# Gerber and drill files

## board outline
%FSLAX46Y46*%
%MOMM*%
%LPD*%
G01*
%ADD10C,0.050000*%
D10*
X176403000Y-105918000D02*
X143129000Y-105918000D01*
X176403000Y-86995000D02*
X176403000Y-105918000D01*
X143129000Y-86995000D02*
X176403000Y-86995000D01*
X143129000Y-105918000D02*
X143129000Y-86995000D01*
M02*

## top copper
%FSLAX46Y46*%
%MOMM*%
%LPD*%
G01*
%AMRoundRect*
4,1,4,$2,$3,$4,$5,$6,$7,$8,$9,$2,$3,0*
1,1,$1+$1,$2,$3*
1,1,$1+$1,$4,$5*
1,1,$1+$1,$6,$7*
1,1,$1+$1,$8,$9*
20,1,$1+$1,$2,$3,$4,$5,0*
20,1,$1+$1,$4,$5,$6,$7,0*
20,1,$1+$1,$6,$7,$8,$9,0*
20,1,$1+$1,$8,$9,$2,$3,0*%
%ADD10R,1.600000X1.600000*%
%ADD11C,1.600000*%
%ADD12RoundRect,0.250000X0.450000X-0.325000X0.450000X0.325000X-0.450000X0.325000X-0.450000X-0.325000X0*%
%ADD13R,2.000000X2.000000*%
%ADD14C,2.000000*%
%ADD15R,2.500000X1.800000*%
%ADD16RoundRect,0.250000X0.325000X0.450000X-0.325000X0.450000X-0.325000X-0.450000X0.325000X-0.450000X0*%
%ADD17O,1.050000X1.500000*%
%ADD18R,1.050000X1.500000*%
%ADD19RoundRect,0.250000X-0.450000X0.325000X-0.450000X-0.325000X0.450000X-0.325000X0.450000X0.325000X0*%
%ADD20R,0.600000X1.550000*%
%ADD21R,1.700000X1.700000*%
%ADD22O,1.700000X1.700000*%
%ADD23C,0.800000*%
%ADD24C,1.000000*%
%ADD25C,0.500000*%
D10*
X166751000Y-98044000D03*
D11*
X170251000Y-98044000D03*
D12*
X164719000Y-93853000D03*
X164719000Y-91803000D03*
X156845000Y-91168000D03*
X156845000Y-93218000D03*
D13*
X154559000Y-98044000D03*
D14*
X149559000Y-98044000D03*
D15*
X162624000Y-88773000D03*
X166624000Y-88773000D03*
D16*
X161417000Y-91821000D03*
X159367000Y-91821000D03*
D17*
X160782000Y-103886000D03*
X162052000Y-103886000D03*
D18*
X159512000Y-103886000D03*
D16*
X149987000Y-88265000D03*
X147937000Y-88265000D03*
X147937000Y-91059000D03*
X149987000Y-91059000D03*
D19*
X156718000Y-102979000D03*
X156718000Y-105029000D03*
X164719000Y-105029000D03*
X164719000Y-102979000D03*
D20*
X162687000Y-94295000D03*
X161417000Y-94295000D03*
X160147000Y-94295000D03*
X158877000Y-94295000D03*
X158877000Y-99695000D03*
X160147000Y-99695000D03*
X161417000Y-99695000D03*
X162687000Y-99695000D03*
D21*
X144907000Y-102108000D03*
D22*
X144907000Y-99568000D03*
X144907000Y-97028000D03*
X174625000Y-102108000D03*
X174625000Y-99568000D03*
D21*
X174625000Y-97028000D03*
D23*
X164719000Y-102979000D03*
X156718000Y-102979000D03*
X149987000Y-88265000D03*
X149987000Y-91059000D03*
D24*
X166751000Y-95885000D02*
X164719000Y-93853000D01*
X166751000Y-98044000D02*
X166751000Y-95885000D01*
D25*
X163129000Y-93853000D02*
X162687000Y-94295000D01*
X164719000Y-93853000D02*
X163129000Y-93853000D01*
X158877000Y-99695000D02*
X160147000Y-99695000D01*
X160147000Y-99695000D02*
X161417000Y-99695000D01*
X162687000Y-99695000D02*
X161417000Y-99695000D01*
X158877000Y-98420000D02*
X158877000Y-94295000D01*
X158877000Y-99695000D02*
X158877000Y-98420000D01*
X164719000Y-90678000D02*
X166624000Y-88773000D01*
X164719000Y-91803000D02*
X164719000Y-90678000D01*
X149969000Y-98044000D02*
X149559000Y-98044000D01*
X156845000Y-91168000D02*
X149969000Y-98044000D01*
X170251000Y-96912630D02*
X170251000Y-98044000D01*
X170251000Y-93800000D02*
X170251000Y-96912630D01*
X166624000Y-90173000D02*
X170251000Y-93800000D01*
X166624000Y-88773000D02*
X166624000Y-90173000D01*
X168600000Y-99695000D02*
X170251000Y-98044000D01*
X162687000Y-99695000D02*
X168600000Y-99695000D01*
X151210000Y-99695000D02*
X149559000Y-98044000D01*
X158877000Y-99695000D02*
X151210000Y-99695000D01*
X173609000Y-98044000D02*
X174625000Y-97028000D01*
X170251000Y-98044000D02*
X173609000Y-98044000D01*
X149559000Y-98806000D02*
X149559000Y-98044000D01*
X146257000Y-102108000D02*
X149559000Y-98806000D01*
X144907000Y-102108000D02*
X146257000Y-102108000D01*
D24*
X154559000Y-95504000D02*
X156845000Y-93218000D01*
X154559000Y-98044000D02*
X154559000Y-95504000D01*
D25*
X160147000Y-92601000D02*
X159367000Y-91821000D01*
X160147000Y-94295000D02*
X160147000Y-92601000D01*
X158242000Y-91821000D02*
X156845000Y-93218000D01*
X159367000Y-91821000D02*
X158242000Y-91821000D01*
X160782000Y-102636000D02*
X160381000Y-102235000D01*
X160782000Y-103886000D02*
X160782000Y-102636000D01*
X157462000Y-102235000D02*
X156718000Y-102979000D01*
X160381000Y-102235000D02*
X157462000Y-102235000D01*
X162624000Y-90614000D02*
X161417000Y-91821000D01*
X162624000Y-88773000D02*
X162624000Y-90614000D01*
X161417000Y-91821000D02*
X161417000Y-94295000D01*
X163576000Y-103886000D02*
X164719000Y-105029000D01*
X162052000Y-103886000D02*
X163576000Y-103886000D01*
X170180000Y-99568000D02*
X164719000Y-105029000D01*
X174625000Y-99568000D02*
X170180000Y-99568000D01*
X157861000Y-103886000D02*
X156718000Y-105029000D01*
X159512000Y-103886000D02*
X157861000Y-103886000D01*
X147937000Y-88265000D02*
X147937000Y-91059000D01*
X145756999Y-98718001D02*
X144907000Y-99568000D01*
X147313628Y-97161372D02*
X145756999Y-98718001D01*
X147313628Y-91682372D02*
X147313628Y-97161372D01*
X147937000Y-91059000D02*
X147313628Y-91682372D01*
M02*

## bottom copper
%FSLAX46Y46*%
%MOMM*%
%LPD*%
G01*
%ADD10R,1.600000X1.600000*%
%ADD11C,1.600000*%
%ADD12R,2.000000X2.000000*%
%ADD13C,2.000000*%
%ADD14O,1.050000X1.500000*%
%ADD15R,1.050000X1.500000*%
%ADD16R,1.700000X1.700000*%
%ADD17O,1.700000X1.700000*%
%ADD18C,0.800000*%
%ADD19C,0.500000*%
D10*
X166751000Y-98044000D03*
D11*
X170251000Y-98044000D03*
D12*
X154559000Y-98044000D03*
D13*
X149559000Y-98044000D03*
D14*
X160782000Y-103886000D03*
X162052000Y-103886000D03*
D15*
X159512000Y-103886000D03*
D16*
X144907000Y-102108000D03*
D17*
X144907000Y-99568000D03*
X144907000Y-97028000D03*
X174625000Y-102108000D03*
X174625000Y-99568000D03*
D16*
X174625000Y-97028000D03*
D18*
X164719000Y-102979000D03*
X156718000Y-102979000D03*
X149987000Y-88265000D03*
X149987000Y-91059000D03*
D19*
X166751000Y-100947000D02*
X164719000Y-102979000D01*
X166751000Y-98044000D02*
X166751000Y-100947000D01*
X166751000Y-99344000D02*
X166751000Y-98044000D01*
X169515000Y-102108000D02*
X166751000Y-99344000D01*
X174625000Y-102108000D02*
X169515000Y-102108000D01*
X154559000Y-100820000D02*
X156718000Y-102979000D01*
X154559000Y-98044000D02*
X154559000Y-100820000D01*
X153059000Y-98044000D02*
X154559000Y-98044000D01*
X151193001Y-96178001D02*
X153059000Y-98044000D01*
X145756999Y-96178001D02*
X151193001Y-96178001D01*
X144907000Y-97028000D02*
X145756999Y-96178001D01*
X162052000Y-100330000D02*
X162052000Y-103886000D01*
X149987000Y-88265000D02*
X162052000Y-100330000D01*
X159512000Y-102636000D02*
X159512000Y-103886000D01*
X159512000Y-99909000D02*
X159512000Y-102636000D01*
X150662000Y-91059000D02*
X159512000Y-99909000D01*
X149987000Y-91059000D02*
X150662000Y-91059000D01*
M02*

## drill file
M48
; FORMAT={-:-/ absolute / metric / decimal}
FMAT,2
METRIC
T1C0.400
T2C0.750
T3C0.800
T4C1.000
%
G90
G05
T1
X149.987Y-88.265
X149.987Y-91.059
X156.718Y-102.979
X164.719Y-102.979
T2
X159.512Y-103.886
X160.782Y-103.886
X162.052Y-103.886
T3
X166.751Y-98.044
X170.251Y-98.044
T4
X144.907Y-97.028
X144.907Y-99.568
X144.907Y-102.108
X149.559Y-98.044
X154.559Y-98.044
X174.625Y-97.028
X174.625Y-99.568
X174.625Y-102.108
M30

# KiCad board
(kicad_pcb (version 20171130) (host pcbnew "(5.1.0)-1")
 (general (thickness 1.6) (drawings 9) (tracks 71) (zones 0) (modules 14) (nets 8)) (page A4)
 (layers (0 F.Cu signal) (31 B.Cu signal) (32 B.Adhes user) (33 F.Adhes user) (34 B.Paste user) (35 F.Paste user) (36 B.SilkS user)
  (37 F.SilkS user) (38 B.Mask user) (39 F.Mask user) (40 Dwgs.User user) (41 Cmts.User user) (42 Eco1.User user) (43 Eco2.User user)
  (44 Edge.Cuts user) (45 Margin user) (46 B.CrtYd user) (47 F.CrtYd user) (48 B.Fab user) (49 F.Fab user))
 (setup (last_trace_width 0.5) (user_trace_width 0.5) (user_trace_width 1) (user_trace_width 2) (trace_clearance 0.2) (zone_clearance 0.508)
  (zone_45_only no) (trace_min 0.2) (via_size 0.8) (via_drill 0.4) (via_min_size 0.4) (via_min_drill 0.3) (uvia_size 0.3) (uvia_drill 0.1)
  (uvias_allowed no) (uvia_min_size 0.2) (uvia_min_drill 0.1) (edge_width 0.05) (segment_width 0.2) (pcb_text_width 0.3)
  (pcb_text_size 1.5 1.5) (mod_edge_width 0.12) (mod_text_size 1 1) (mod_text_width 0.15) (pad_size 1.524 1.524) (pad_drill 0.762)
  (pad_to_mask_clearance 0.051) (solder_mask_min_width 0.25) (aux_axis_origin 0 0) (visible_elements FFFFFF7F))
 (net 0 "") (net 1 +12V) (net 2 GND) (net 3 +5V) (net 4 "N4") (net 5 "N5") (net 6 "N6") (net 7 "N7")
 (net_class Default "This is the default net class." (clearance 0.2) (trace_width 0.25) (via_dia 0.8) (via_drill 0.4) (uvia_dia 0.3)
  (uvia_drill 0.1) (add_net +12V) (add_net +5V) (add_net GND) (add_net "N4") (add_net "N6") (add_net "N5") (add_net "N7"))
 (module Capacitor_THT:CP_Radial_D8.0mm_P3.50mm (layer F.Cu) (at 166.751 98.044)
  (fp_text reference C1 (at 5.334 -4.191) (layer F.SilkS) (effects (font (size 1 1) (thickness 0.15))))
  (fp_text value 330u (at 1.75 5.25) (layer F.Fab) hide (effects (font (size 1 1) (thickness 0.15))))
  (pad 1 thru_hole rect (at 0 0) (size 1.6 1.6) (drill 0.8) (layers *.Cu *.Mask) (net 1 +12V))
  (pad 2 thru_hole circle (at 3.5 0) (size 1.6 1.6) (drill 0.8) (layers *.Cu *.Mask) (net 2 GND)))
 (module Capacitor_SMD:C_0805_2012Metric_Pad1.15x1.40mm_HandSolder (layer F.Cu) (at 164.719 92.828 90)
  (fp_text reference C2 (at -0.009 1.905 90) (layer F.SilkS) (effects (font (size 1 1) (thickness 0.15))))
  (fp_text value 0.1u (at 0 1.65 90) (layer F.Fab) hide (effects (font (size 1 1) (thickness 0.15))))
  (pad 1 smd roundrect (at -1.025 0 90) (size 1.15 1.4) (layers F.Cu F.Paste F.Mask) (roundrect_rratio 0.217391) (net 1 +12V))
  (pad 2 smd roundrect (at 1.025 0 90) (size 1.15 1.4) (layers F.Cu F.Paste F.Mask) (roundrect_rratio 0.217391) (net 2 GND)))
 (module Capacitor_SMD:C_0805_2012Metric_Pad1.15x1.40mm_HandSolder (layer F.Cu) (at 156.845 92.193 90)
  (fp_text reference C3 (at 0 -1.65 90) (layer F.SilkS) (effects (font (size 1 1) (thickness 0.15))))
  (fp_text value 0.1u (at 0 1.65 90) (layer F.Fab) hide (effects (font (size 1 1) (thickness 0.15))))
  (pad 2 smd roundrect (at 1.025 0 90) (size 1.15 1.4) (layers F.Cu F.Paste F.Mask) (roundrect_rratio 0.217391) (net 2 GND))
  (pad 1 smd roundrect (at -1.025 0 90) (size 1.15 1.4) (layers F.Cu F.Paste F.Mask) (roundrect_rratio 0.217391) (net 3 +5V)))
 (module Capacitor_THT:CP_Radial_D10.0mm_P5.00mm (layer F.Cu) (at 154.559 98.044 180)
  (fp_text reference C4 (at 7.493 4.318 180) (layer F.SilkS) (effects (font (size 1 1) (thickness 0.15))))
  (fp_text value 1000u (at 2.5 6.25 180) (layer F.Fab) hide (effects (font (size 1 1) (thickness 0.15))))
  (pad 1 thru_hole rect (at 0 0 180) (size 2 2) (drill 1) (layers *.Cu *.Mask) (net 3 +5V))
  (pad 2 thru_hole circle (at 5 0 180) (size 2 2) (drill 1) (layers *.Cu *.Mask) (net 2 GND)))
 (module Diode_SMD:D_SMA (layer F.Cu) (at 164.624 88.773)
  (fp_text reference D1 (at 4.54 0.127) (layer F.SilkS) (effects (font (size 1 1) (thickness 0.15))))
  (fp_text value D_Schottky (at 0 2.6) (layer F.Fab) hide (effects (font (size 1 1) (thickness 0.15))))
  (pad 1 smd rect (at -2 0) (size 2.5 1.8) (layers F.Cu F.Paste F.Mask) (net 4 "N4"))
  (pad 2 smd rect (at 2 0) (size 2.5 1.8) (layers F.Cu F.Paste F.Mask) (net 2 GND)))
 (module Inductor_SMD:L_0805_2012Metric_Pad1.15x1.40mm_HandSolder (layer F.Cu) (at 160.392 91.821 180)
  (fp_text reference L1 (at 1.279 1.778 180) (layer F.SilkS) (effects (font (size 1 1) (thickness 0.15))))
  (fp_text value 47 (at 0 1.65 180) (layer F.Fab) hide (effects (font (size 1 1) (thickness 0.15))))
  (pad 1 smd roundrect (at -1.025 0 180) (size 1.15 1.4) (layers F.Cu F.Paste F.Mask) (roundrect_rratio 0.217391) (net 4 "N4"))
  (pad 2 smd roundrect (at 1.025 0 180) (size 1.15 1.4) (layers F.Cu F.Paste F.Mask) (roundrect_rratio 0.217391) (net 3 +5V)))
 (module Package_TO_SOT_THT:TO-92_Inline (layer F.Cu) (at 159.512 103.886)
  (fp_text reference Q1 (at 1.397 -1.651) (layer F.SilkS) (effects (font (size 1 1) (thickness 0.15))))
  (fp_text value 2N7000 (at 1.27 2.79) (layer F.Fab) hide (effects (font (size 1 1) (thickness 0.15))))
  (pad 2 thru_hole oval (at 1.27 0) (size 1.05 1.5) (drill 0.75) (layers *.Cu *.Mask) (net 3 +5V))
  (pad 3 thru_hole oval (at 2.54 0) (size 1.05 1.5) (drill 0.75) (layers *.Cu *.Mask) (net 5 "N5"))
  (pad 1 thru_hole rect (at 0 0) (size 1.05 1.5) (drill 0.75) (layers *.Cu *.Mask) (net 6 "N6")))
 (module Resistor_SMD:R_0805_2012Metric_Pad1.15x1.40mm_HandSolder (layer F.Cu) (at 148.962 88.265 180)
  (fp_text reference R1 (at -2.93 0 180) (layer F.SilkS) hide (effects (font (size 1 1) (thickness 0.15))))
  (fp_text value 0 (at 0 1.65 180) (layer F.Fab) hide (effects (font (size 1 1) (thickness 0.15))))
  (pad 1 smd roundrect (at -1.025 0 180) (size 1.15 1.4) (layers F.Cu F.Paste F.Mask) (roundrect_rratio 0.217391) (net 5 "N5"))
  (pad 2 smd roundrect (at 1.025 0 180) (size 1.15 1.4) (layers F.Cu F.Paste F.Mask) (roundrect_rratio 0.217391) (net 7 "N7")))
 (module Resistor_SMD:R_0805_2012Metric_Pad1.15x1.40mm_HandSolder (layer F.Cu) (at 148.962 91.059 180)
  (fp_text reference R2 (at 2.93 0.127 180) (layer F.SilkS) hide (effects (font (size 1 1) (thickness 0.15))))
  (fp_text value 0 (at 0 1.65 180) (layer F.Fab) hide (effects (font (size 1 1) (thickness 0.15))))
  (pad 2 smd roundrect (at 1.025 0 180) (size 1.15 1.4) (layers F.Cu F.Paste F.Mask) (roundrect_rratio 0.217391) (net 7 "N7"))
  (pad 1 smd roundrect (at -1.025 0 180) (size 1.15 1.4) (layers F.Cu F.Paste F.Mask) (roundrect_rratio 0.217391) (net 6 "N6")))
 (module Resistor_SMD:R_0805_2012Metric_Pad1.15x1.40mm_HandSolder (layer F.Cu) (at 156.718 104.004 270)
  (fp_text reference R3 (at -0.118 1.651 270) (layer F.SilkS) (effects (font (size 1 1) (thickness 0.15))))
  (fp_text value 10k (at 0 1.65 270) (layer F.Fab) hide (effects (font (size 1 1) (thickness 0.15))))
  (pad 1 smd roundrect (at -1.025 0 270) (size 1.15 1.4) (layers F.Cu F.Paste F.Mask) (roundrect_rratio 0.217391) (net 3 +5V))
  (pad 2 smd roundrect (at 1.025 0 270) (size 1.15 1.4) (layers F.Cu F.Paste F.Mask) (roundrect_rratio 0.217391) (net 6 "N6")))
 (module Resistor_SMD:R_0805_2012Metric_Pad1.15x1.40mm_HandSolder (layer F.Cu) (at 164.719 104.004 270)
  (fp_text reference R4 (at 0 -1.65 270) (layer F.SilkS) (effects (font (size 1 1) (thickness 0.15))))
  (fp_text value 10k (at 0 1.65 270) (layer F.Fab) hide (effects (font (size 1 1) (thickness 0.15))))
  (pad 2 smd roundrect (at 1.025 0 270) (size 1.15 1.4) (layers F.Cu F.Paste F.Mask) (roundrect_rratio 0.217391) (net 5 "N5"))
  (pad 1 smd roundrect (at -1.025 0 270) (size 1.15 1.4) (layers F.Cu F.Paste F.Mask) (roundrect_rratio 0.217391) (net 1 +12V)))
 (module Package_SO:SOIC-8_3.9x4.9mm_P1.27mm (layer F.Cu) (at 160.782 96.995 270)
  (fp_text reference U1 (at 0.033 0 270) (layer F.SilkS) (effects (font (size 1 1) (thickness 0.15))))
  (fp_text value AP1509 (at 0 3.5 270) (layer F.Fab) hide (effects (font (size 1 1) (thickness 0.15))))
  (pad 1 smd rect (at -2.7 -1.905 270) (size 1.55 0.6) (layers F.Cu F.Paste F.Mask) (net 1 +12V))
  (pad 2 smd rect (at -2.7 -0.635 270) (size 1.55 0.6) (layers F.Cu F.Paste F.Mask) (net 4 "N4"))
  (pad 3 smd rect (at -2.7 0.635 270) (size 1.55 0.6) (layers F.Cu F.Paste F.Mask) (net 3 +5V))
  (pad 4 smd rect (at -2.7 1.905 270) (size 1.55 0.6) (layers F.Cu F.Paste F.Mask) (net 2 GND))
  (pad 5 smd rect (at 2.7 1.905 270) (size 1.55 0.6) (layers F.Cu F.Paste F.Mask) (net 2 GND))
  (pad 6 smd rect (at 2.7 0.635 270) (size 1.55 0.6) (layers F.Cu F.Paste F.Mask) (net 2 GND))
  (pad 7 smd rect (at 2.7 -0.635 270) (size 1.55 0.6) (layers F.Cu F.Paste F.Mask) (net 2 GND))
  (pad 8 smd rect (at 2.7 -1.905 270) (size 1.55 0.6) (layers F.Cu F.Paste F.Mask) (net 2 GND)))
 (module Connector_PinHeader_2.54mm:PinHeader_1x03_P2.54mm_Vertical (layer F.Cu) (at 144.907 102.108 180)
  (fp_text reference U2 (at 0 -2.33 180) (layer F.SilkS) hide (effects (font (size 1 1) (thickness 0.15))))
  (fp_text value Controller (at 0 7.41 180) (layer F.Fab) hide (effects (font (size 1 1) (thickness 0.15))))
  (pad 1 thru_hole rect (at 0 0 180) (size 1.7 1.7) (drill 1) (layers *.Cu *.Mask) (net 2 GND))
  (pad 2 thru_hole oval (at 0 2.54 180) (size 1.7 1.7) (drill 1) (layers *.Cu *.Mask) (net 7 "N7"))
  (pad 3 thru_hole oval (at 0 5.08 180) (size 1.7 1.7) (drill 1) (layers *.Cu *.Mask) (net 3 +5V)))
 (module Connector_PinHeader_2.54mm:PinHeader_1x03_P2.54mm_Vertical (layer F.Cu) (at 174.625 97.028)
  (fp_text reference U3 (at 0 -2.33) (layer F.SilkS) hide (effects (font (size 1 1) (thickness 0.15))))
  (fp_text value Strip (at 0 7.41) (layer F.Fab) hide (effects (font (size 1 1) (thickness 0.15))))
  (pad 3 thru_hole oval (at 0 5.08) (size 1.7 1.7) (drill 1) (layers *.Cu *.Mask) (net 1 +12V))
  (pad 2 thru_hole oval (at 0 2.54) (size 1.7 1.7) (drill 1) (layers *.Cu *.Mask) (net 5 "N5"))
  (pad 1 thru_hole rect (at 0 0) (size 1.7 1.7) (drill 1) (layers *.Cu *.Mask) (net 2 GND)))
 (gr_line (start 176.403 105.918) (end 143.129 105.918) (layer Edge.Cuts) (width 0.05))
 (gr_line (start 176.403 86.995) (end 176.403 105.918) (layer Edge.Cuts) (width 0.05))
 (gr_line (start 143.129 86.995) (end 176.403 86.995) (layer Edge.Cuts) (width 0.05))
 (gr_line (start 143.129 105.918) (end 143.129 86.995) (layer Edge.Cuts) (width 0.05))
 (segment (start 166.751 95.885) (end 164.719 93.853) (width 1) (layer F.Cu) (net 1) (status 20))
 (segment (start 166.751 98.044) (end 166.751 95.885) (width 1) (layer F.Cu) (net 1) (status 10))
 (segment (start 163.129 93.853) (end 162.687 94.295) (width 0.5) (layer F.Cu) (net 1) (status 20))
 (segment (start 164.719 93.853) (end 163.129 93.853) (width 0.5) (layer F.Cu) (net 1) (status 10))
 (via (at 164.719 102.979) (size 0.8) (drill 0.4) (layers F.Cu B.Cu) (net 1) (status 30))
 (segment (start 166.751 100.947) (end 164.719 102.979) (width 0.5) (layer B.Cu) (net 1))
 (segment (start 166.751 98.044) (end 166.751 100.947) (width 0.5) (layer B.Cu) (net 1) (status 10))
 (segment (start 166.751 99.344) (end 166.751 98.044) (width 0.5) (layer B.Cu) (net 1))
 (segment (start 169.515 102.108) (end 166.751 99.344) (width 0.5) (layer B.Cu) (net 1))
 (segment (start 174.625 102.108) (end 169.515 102.108) (width 0.5) (layer B.Cu) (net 1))
 (segment (start 158.877 99.695) (end 160.147 99.695) (width 0.5) (layer F.Cu) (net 2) (status 30))
 (segment (start 160.147 99.695) (end 161.417 99.695) (width 0.5) (layer F.Cu) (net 2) (status 30))
 (segment (start 162.687 99.695) (end 161.417 99.695) (width 0.5) (layer F.Cu) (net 2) (status 30))
 (segment (start 158.877 98.42) (end 158.877 94.295) (width 0.5) (layer F.Cu) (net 2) (status 20))
 (segment (start 158.877 99.695) (end 158.877 98.42) (width 0.5) (layer F.Cu) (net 2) (status 10))
 (segment (start 164.719 90.678) (end 166.624 88.773) (width 0.5) (layer F.Cu) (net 2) (status 20))
 (segment (start 164.719 91.803) (end 164.719 90.678) (width 0.5) (layer F.Cu) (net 2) (status 10))
 (segment (start 149.969 98.044) (end 149.559 98.044) (width 0.5) (layer F.Cu) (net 2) (status 30))
 (segment (start 156.845 91.168) (end 149.969 98.044) (width 0.5) (layer F.Cu) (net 2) (status 30))
 (segment (start 170.251 96.91263) (end 170.251 98.044) (width 0.5) (layer F.Cu) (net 2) (status 20))
 (segment (start 170.251 93.8) (end 170.251 96.91263) (width 0.5) (layer F.Cu) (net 2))
 (segment (start 166.624 90.173) (end 170.251 93.8) (width 0.5) (layer F.Cu) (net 2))
 (segment (start 166.624 88.773) (end 166.624 90.173) (width 0.5) (layer F.Cu) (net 2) (status 10))
 (segment (start 168.6 99.695) (end 170.251 98.044) (width 0.5) (layer F.Cu) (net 2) (status 20))
 (segment (start 162.687 99.695) (end 168.6 99.695) (width 0.5) (layer F.Cu) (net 2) (status 10))
 (segment (start 151.21 99.695) (end 149.559 98.044) (width 0.5) (layer F.Cu) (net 2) (status 20))
 (segment (start 158.877 99.695) (end 151.21 99.695) (width 0.5) (layer F.Cu) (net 2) (status 10))
 (segment (start 173.609 98.044) (end 174.625 97.028) (width 0.5) (layer F.Cu) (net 2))
 (segment (start 170.251 98.044) (end 173.609 98.044) (width 0.5) (layer F.Cu) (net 2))
 (segment (start 149.559 98.806) (end 149.559 98.044) (width 0.5) (layer F.Cu) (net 2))
 (segment (start 146.257 102.108) (end 149.559 98.806) (width 0.5) (layer F.Cu) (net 2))
 (segment (start 144.907 102.108) (end 146.257 102.108) (width 0.5) (layer F.Cu) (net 2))
 (segment (start 154.559 95.504) (end 156.845 93.218) (width 1) (layer F.Cu) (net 3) (status 20))
 (segment (start 154.559 98.044) (end 154.559 95.504) (width 1) (layer F.Cu) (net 3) (status 10))
 (segment (start 160.147 92.601) (end 159.367 91.821) (width 0.5) (layer F.Cu) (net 3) (status 20))
 (segment (start 160.147 94.295) (end 160.147 92.601) (width 0.5) (layer F.Cu) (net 3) (status 10))
 (segment (start 158.242 91.821) (end 156.845 93.218) (width 0.5) (layer F.Cu) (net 3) (status 20))
 (segment (start 159.367 91.821) (end 158.242 91.821) (width 0.5) (layer F.Cu) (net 3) (status 10))
 (via (at 156.718 102.979) (size 0.8) (drill 0.4) (layers F.Cu B.Cu) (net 3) (status 30))
 (segment (start 154.559 100.82) (end 156.718 102.979) (width 0.5) (layer B.Cu) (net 3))
 (segment (start 154.559 98.044) (end 154.559 100.82) (width 0.5) (layer B.Cu) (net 3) (status 10))
 (segment (start 153.059 98.044) (end 154.559 98.044) (width 0.5) (layer B.Cu) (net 3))
 (segment (start 151.193001 96.178001) (end 153.059 98.044) (width 0.5) (layer B.Cu) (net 3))
 (segment (start 145.756999 96.178001) (end 151.193001 96.178001) (width 0.5) (layer B.Cu) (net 3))
 (segment (start 144.907 97.028) (end 145.756999 96.178001) (width 0.5) (layer B.Cu) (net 3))
 (segment (start 160.782 102.636) (end 160.381 102.235) (width 0.5) (layer F.Cu) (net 3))
 (segment (start 160.782 103.886) (end 160.782 102.636) (width 0.5) (layer F.Cu) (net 3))
 (segment (start 157.462 102.235) (end 156.718 102.979) (width 0.5) (layer F.Cu) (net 3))
 (segment (start 160.381 102.235) (end 157.462 102.235) (width 0.5) (layer F.Cu) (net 3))
 (segment (start 162.624 90.614) (end 161.417 91.821) (width 0.5) (layer F.Cu) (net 4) (status 20))
 (segment (start 162.624 88.773) (end 162.624 90.614) (width 0.5) (layer F.Cu) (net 4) (status 10))
 (segment (start 161.417 91.821) (end 161.417 94.295) (width 0.5) (layer F.Cu) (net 4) (status 30))
 (segment (start 163.576 103.886) (end 164.719 105.029) (width 0.5) (layer F.Cu) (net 5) (status 20))
 (segment (start 162.052 103.886) (end 163.576 103.886) (width 0.5) (layer F.Cu) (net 5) (status 10))
 (segment (start 170.18 99.568) (end 164.719 105.029) (width 0.5) (layer F.Cu) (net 5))
 (segment (start 174.625 99.568) (end 170.18 99.568) (width 0.5) (layer F.Cu) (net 5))
 (via (at 149.987 88.265) (size 0.8) (drill 0.4) (layers F.Cu B.Cu) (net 5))
 (segment (start 162.052 100.33) (end 162.052 103.886) (width 0.5) (layer B.Cu) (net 5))
 (segment (start 149.987 88.265) (end 162.052 100.33) (width 0.5) (layer B.Cu) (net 5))
 (segment (start 157.861 103.886) (end 156.718 105.029) (width 0.5) (layer F.Cu) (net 6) (status 20))
 (segment (start 159.512 103.886) (end 157.861 103.886) (width 0.5) (layer F.Cu) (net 6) (status 10))
 (via (at 149.987 91.059) (size 0.8) (drill 0.4) (layers F.Cu B.Cu) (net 6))
 (segment (start 159.512 102.636) (end 159.512 103.886) (width 0.5) (layer B.Cu) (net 6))
 (segment (start 159.512 99.909) (end 159.512 102.636) (width 0.5) (layer B.Cu) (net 6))
 (segment (start 150.662 91.059) (end 159.512 99.909) (width 0.5) (layer B.Cu) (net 6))
 (segment (start 149.987 91.059) (end 150.662 91.059) (width 0.5) (layer B.Cu) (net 6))
 (segment (start 147.937 88.265) (end 147.937 91.059) (width 0.5) (layer F.Cu) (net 7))
 (segment (start 145.756999 98.718001) (end 144.907 99.568) (width 0.5) (layer F.Cu) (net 7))
 (segment (start 147.313628 97.161372) (end 145.756999 98.718001) (width 0.5) (layer F.Cu) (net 7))
 (segment (start 147.313628 91.682372) (end 147.313628 97.161372) (width 0.5) (layer F.Cu) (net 7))
 (segment (start 147.937 91.059) (end 147.313628 91.682372) (width 0.5) (layer F.Cu) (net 7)))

